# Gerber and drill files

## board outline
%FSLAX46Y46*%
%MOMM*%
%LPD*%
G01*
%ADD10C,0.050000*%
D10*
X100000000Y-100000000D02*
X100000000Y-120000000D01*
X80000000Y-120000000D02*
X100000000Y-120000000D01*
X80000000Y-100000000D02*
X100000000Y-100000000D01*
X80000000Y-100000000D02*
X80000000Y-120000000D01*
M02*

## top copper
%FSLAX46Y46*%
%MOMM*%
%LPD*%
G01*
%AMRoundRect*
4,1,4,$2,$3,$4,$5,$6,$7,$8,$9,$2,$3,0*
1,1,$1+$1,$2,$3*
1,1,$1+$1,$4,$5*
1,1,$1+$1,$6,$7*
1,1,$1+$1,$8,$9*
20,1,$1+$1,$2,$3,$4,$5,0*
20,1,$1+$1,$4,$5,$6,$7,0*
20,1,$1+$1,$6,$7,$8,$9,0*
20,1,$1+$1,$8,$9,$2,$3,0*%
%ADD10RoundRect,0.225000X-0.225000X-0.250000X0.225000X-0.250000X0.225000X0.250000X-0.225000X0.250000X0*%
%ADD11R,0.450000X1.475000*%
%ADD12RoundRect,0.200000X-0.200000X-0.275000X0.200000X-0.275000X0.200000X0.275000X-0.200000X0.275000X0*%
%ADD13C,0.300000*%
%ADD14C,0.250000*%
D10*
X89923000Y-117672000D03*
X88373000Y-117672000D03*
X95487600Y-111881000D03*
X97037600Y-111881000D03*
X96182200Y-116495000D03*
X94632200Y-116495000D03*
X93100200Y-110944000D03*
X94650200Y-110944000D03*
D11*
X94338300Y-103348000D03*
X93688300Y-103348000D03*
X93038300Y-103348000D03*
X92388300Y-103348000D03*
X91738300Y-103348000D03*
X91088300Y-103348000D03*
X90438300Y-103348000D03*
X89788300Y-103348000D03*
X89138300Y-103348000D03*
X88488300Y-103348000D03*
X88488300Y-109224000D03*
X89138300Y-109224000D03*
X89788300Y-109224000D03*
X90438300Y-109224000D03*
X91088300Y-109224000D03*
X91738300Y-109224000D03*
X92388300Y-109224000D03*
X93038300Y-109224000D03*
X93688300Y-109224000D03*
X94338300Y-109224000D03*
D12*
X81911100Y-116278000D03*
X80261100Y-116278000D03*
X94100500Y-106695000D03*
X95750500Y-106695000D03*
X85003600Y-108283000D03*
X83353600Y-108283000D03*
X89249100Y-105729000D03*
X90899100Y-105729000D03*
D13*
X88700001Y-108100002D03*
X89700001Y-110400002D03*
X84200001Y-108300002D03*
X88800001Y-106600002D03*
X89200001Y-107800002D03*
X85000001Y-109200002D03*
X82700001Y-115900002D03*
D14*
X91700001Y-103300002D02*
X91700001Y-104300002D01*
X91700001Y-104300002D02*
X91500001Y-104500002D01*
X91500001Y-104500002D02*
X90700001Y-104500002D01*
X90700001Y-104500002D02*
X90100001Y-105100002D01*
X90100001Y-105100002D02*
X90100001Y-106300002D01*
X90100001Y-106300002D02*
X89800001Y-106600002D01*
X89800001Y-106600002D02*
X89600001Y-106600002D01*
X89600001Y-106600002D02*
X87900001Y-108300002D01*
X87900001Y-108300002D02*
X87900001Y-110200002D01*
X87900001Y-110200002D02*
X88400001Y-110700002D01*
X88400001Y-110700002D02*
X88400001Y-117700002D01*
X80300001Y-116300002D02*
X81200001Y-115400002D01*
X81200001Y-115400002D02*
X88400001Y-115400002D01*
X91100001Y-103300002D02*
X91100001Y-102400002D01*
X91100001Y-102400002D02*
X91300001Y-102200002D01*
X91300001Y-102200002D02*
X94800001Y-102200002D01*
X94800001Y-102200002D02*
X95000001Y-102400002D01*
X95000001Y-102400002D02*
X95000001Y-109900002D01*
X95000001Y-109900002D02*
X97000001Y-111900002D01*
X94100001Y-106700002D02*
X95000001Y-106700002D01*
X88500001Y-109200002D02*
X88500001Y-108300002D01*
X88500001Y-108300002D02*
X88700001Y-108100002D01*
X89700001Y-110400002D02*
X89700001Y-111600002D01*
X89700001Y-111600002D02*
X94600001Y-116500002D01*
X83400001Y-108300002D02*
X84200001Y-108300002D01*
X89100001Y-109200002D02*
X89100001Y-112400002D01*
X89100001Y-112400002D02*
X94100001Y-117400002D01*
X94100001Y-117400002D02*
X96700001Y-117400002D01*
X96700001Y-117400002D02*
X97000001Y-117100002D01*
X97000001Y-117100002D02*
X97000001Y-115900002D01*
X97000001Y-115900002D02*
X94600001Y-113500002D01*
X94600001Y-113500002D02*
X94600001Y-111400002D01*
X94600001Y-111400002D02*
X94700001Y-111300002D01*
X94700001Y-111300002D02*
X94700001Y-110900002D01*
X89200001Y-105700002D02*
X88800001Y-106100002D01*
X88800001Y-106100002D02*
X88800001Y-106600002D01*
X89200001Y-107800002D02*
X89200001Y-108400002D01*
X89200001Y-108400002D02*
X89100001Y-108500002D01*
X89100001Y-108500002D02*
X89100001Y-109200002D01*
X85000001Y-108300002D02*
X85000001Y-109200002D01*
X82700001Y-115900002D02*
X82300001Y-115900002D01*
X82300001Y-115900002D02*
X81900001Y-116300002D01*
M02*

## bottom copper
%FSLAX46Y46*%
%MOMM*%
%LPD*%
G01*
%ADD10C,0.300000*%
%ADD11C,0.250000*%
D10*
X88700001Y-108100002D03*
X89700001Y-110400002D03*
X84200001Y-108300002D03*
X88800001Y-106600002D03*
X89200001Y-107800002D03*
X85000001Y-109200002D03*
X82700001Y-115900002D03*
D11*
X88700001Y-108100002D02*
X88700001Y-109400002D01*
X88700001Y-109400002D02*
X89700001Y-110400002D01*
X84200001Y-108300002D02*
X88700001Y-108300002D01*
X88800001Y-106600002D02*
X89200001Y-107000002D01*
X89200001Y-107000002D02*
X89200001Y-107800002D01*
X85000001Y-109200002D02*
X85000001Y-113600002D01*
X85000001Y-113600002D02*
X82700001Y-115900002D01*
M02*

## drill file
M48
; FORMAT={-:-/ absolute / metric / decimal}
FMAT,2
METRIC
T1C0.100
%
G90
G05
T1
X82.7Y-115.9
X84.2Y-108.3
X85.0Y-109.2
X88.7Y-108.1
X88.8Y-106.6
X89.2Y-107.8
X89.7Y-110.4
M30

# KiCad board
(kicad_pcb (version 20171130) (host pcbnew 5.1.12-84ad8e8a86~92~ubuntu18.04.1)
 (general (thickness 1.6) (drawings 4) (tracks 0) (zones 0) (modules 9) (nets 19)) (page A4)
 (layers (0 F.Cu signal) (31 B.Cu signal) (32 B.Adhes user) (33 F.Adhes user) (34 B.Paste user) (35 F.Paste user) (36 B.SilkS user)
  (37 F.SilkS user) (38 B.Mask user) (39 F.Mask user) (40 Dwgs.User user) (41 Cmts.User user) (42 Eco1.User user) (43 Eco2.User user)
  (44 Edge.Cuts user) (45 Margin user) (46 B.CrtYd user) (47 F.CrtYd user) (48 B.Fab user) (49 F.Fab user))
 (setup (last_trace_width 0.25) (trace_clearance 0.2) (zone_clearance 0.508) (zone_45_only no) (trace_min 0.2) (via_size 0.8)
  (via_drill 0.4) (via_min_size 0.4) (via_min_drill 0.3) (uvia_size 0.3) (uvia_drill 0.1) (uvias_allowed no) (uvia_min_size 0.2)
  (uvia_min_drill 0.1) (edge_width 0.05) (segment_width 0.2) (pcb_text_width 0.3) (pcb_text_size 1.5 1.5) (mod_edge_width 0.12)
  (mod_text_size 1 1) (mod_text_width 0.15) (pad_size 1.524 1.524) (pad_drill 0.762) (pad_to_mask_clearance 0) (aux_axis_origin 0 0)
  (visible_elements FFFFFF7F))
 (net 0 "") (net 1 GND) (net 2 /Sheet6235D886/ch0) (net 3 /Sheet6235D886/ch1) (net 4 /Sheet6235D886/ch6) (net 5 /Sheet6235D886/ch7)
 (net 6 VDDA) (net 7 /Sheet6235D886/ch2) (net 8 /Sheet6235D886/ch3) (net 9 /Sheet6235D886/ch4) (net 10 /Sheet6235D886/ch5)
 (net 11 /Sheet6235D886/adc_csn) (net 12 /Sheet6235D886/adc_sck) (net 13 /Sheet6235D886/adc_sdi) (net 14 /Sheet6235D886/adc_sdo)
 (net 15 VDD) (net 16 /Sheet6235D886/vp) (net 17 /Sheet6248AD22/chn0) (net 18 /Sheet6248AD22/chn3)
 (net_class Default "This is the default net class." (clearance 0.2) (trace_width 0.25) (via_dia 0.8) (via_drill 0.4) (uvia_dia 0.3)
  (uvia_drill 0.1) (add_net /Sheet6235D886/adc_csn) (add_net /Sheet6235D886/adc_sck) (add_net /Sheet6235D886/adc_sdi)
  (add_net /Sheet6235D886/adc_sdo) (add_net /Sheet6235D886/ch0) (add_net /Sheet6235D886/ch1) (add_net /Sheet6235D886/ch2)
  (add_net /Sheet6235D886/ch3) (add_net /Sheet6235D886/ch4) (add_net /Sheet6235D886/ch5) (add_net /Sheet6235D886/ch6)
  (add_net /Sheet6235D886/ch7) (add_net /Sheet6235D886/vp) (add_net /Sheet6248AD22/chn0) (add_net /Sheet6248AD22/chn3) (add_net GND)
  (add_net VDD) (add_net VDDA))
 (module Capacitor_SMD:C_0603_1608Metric (layer F.Cu) (at 89.148000 117.672000)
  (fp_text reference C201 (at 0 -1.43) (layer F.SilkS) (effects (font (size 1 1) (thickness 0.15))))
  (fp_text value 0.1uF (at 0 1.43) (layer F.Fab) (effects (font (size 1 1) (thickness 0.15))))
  (pad 2 smd roundrect (at 0.775 0) (size 0.9 0.95) (layers F.Cu F.Mask F.Paste) (roundrect_rratio 0.25) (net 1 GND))
  (pad 1 smd roundrect (at -0.775 0) (size 0.9 0.95) (layers F.Cu F.Mask F.Paste) (roundrect_rratio 0.25) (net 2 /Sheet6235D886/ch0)))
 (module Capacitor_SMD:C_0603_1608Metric (layer F.Cu) (at 96.262600 111.881000)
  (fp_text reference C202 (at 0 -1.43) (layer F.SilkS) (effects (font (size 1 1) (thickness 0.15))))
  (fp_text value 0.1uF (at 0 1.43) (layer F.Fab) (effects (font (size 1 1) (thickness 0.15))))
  (pad 1 smd roundrect (at -0.775 0) (size 0.9 0.95) (layers F.Cu F.Mask F.Paste) (roundrect_rratio 0.25) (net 1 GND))
  (pad 2 smd roundrect (at 0.775 0) (size 0.9 0.95) (layers F.Cu F.Mask F.Paste) (roundrect_rratio 0.25) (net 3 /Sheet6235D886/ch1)))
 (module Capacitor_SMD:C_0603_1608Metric (layer F.Cu) (at 95.407200 116.495000)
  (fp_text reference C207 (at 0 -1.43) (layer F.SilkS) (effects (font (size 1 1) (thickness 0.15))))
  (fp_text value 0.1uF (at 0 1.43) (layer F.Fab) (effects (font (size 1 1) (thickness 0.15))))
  (pad 2 smd roundrect (at 0.775 0) (size 0.9 0.95) (layers F.Cu F.Mask F.Paste) (roundrect_rratio 0.25) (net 1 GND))
  (pad 1 smd roundrect (at -0.775 0) (size 0.9 0.95) (layers F.Cu F.Mask F.Paste) (roundrect_rratio 0.25) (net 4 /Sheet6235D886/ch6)))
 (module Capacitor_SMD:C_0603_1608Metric (layer F.Cu) (at 93.875200 110.944000)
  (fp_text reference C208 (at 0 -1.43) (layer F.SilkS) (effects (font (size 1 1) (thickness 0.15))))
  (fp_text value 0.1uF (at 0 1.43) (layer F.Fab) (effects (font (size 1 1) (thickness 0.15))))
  (pad 1 smd roundrect (at -0.775 0) (size 0.9 0.95) (layers F.Cu F.Mask F.Paste) (roundrect_rratio 0.25) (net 1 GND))
  (pad 2 smd roundrect (at 0.775 0) (size 0.9 0.95) (layers F.Cu F.Mask F.Paste) (roundrect_rratio 0.25) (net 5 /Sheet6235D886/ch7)))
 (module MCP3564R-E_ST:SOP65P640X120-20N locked (layer F.Cu) (at 91.413300 106.286000 270.000000)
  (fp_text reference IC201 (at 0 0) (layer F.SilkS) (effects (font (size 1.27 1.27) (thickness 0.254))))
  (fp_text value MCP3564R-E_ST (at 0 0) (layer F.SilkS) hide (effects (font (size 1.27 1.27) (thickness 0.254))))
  (pad 1 smd rect (at -2.938 -2.925) (size 0.45 1.475) (layers F.Cu F.Mask F.Paste) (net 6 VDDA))
  (pad 2 smd rect (at -2.938 -2.275) (size 0.45 1.475) (layers F.Cu F.Mask F.Paste) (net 1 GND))
  (pad 3 smd rect (at -2.938 -1.625) (size 0.45 1.475) (layers F.Cu F.Mask F.Paste) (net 1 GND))
  (pad 4 smd rect (at -2.938 -0.975) (size 0.45 1.475) (layers F.Cu F.Mask F.Paste))
  (pad 5 smd rect (at -2.938 -0.325) (size 0.45 1.475) (layers F.Cu F.Mask F.Paste) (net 2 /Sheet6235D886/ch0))
  (pad 6 smd rect (at -2.938 0.325) (size 0.45 1.475) (layers F.Cu F.Mask F.Paste) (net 3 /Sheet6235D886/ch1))
  (pad 7 smd rect (at -2.938 0.975) (size 0.45 1.475) (layers F.Cu F.Mask F.Paste) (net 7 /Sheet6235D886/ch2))
  (pad 8 smd rect (at -2.938 1.625) (size 0.45 1.475) (layers F.Cu F.Mask F.Paste) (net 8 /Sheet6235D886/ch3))
  (pad 9 smd rect (at -2.938 2.275) (size 0.45 1.475) (layers F.Cu F.Mask F.Paste) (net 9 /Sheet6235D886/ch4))
  (pad 10 smd rect (at -2.938 2.925) (size 0.45 1.475) (layers F.Cu F.Mask F.Paste) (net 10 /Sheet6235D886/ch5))
  (pad 11 smd rect (at 2.938 2.925) (size 0.45 1.475) (layers F.Cu F.Mask F.Paste) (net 4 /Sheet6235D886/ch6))
  (pad 12 smd rect (at 2.938 2.275) (size 0.45 1.475) (layers F.Cu F.Mask F.Paste) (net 5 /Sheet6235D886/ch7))
  (pad 13 smd rect (at 2.938 1.625) (size 0.45 1.475) (layers F.Cu F.Mask F.Paste) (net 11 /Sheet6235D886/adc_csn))
  (pad 14 smd rect (at 2.938 0.975) (size 0.45 1.475) (layers F.Cu F.Mask F.Paste) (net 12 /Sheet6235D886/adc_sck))
  (pad 15 smd rect (at 2.938 0.325) (size 0.45 1.475) (layers F.Cu F.Mask F.Paste) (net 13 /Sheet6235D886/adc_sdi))
  (pad 16 smd rect (at 2.938 -0.325) (size 0.45 1.475) (layers F.Cu F.Mask F.Paste) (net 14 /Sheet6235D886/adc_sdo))
  (pad 17 smd rect (at 2.938 -0.975) (size 0.45 1.475) (layers F.Cu F.Mask F.Paste))
  (pad 18 smd rect (at 2.938 -1.625) (size 0.45 1.475) (layers F.Cu F.Mask F.Paste))
  (pad 19 smd rect (at 2.938 -2.275) (size 0.45 1.475) (layers F.Cu F.Mask F.Paste) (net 1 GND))
  (pad 20 smd rect (at 2.938 -2.925) (size 0.45 1.475) (layers F.Cu F.Mask F.Paste) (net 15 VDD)))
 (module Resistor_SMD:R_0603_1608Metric (layer F.Cu) (at 81.086100 116.278000)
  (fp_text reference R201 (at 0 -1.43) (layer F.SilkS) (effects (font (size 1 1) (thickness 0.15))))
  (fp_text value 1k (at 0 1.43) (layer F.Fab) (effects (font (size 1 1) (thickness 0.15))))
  (pad 2 smd roundrect (at 0.825 0) (size 0.8 0.95) (layers F.Cu F.Mask F.Paste) (roundrect_rratio 0.25) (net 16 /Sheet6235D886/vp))
  (pad 1 smd roundrect (at -0.825 0) (size 0.8 0.95) (layers F.Cu F.Mask F.Paste) (roundrect_rratio 0.25) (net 2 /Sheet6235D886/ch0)))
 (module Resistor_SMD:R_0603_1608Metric (layer F.Cu) (at 94.925500 106.695000)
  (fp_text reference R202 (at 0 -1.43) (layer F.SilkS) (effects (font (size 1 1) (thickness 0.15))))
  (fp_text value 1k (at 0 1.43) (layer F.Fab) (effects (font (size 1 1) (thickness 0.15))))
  (pad 1 smd roundrect (at -0.825 0) (size 0.8 0.95) (layers F.Cu F.Mask F.Paste) (roundrect_rratio 0.25) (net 3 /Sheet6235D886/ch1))
  (pad 2 smd roundrect (at 0.825 0) (size 0.8 0.95) (layers F.Cu F.Mask F.Paste) (roundrect_rratio 0.25) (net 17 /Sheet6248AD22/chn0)))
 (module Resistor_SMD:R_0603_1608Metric (layer F.Cu) (at 84.178600 108.283000)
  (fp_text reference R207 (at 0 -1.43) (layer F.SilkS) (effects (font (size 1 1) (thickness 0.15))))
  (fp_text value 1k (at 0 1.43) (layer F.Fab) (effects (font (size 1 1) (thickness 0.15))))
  (pad 2 smd roundrect (at 0.825 0) (size 0.8 0.95) (layers F.Cu F.Mask F.Paste) (roundrect_rratio 0.25) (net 16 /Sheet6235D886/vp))
  (pad 1 smd roundrect (at -0.825 0) (size 0.8 0.95) (layers F.Cu F.Mask F.Paste) (roundrect_rratio 0.25) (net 4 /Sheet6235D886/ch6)))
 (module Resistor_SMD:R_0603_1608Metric (layer F.Cu) (at 90.074100 105.729000)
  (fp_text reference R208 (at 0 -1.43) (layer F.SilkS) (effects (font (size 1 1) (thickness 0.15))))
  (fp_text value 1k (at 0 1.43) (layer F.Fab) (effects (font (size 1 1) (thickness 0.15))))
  (pad 1 smd roundrect (at -0.825 0) (size 0.8 0.95) (layers F.Cu F.Mask F.Paste) (roundrect_rratio 0.25) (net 5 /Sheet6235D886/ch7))
  (pad 2 smd roundrect (at 0.825 0) (size 0.8 0.95) (layers F.Cu F.Mask F.Paste) (roundrect_rratio 0.25) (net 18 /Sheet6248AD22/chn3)))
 (gr_line (start 100 100) (end 100 120) (layer Edge.Cuts) (width 0.05))
 (gr_line (start 80 120) (end 100 120) (layer Edge.Cuts) (width 0.05))
 (gr_line (start 80 100) (end 100 100) (layer Edge.Cuts) (width 0.05))
 (gr_line (start 80 100) (end 80 120) (layer Edge.Cuts) (width 0.05))
 (segment (start 91.700001 103.300002) (end 91.700001 104.300002) (width 0.250000) (layer F.Cu) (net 2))
 (segment (start 91.700001 104.300002) (end 91.500001 104.500002) (width 0.250000) (layer F.Cu) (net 2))
 (segment (start 91.500001 104.500002) (end 90.700001 104.500002) (width 0.250000) (layer F.Cu) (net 2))
 (segment (start 90.700001 104.500002) (end 90.100001 105.100002) (width 0.250000) (layer F.Cu) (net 2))
 (segment (start 90.100001 105.100002) (end 90.100001 106.300002) (width 0.250000) (layer F.Cu) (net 2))
 (segment (start 90.100001 106.300002) (end 89.800001 106.600002) (width 0.250000) (layer F.Cu) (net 2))
 (segment (start 89.800001 106.600002) (end 89.600001 106.600002) (width 0.250000) (layer F.Cu) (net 2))
 (segment (start 89.600001 106.600002) (end 87.900001 108.300002) (width 0.250000) (layer F.Cu) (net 2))
 (segment (start 87.900001 108.300002) (end 87.900001 110.200002) (width 0.250000) (layer F.Cu) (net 2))
 (segment (start 87.900001 110.200002) (end 88.400001 110.700002) (width 0.250000) (layer F.Cu) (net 2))
 (segment (start 88.400001 110.700002) (end 88.400001 117.700002) (width 0.250000) (layer F.Cu) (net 2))
 (segment (start 80.300001 116.300002) (end 81.200001 115.400002) (width 0.250000) (layer F.Cu) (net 2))
 (segment (start 81.200001 115.400002) (end 88.400001 115.400002) (width 0.250000) (layer F.Cu) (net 2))
 (segment (start 91.100001 103.300002) (end 91.100001 102.400002) (width 0.250000) (layer F.Cu) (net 3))
 (segment (start 91.100001 102.400002) (end 91.300001 102.200002) (width 0.250000) (layer F.Cu) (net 3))
 (segment (start 91.300001 102.200002) (end 94.800001 102.200002) (width 0.250000) (layer F.Cu) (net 3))
 (segment (start 94.800001 102.200002) (end 95.000001 102.400002) (width 0.250000) (layer F.Cu) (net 3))
 (segment (start 95.000001 102.400002) (end 95.000001 109.900002) (width 0.250000) (layer F.Cu) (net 3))
 (segment (start 95.000001 109.900002) (end 97.000001 111.900002) (width 0.250000) (layer F.Cu) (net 3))
 (segment (start 94.100001 106.700002) (end 95.000001 106.700002) (width 0.250000) (layer F.Cu) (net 3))
 (segment (start 88.500001 109.200002) (end 88.500001 108.300002) (width 0.250000) (layer F.Cu) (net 4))
 (segment (start 88.500001 108.300002) (end 88.700001 108.100002) (width 0.250000) (layer F.Cu) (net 4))
 (segment (start 88.700001 108.100002) (end 88.700001 109.400002) (width 0.250000) (layer B.Cu) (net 4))
 (segment (start 88.700001 109.400002) (end 89.700001 110.400002) (width 0.250000) (layer B.Cu) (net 4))
 (segment (start 89.700001 110.400002) (end 89.700001 111.600002) (width 0.250000) (layer F.Cu) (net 4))
 (segment (start 89.700001 111.600002) (end 94.600001 116.500002) (width 0.250000) (layer F.Cu) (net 4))
 (segment (start 83.400001 108.300002) (end 84.200001 108.300002) (width 0.250000) (layer F.Cu) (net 4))
 (segment (start 84.200001 108.300002) (end 88.700001 108.300002) (width 0.250000) (layer B.Cu) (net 4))
 (via micro (at 88.700001 108.100002) (size 0.300000) (drill 0.100000) (layers F.Cu B.Cu) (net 4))
 (via micro (at 89.700001 110.400002) (size 0.300000) (drill 0.100000) (layers F.Cu B.Cu) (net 4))
 (via micro (at 84.200001 108.300002) (size 0.300000) (drill 0.100000) (layers F.Cu B.Cu) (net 4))
 (segment (start 89.100001 109.200002) (end 89.100001 112.400002) (width 0.250000) (layer F.Cu) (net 5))
 (segment (start 89.100001 112.400002) (end 94.100001 117.400002) (width 0.250000) (layer F.Cu) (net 5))
 (segment (start 94.100001 117.400002) (end 96.700001 117.400002) (width 0.250000) (layer F.Cu) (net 5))
 (segment (start 96.700001 117.400002) (end 97.000001 117.100002) (width 0.250000) (layer F.Cu) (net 5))
 (segment (start 97.000001 117.100002) (end 97.000001 115.900002) (width 0.250000) (layer F.Cu) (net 5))
 (segment (start 97.000001 115.900002) (end 94.600001 113.500002) (width 0.250000) (layer F.Cu) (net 5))
 (segment (start 94.600001 113.500002) (end 94.600001 111.400002) (width 0.250000) (layer F.Cu) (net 5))
 (segment (start 94.600001 111.400002) (end 94.700001 111.300002) (width 0.250000) (layer F.Cu) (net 5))
 (segment (start 94.700001 111.300002) (end 94.700001 110.900002) (width 0.250000) (layer F.Cu) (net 5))
 (segment (start 89.200001 105.700002) (end 88.800001 106.100002) (width 0.250000) (layer F.Cu) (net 5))
 (segment (start 88.800001 106.100002) (end 88.800001 106.600002) (width 0.250000) (layer F.Cu) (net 5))
 (segment (start 88.800001 106.600002) (end 89.200001 107.000002) (width 0.250000) (layer B.Cu) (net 5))
 (segment (start 89.200001 107.000002) (end 89.200001 107.800002) (width 0.250000) (layer B.Cu) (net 5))
 (segment (start 89.200001 107.800002) (end 89.200001 108.400002) (width 0.250000) (layer F.Cu) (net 5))
 (segment (start 89.200001 108.400002) (end 89.100001 108.500002) (width 0.250000) (layer F.Cu) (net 5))
 (segment (start 89.100001 108.500002) (end 89.100001 109.200002) (width 0.250000) (layer F.Cu) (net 5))
 (via micro (at 88.800001 106.600002) (size 0.300000) (drill 0.100000) (layers F.Cu B.Cu) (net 5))
 (via micro (at 89.200001 107.800002) (size 0.300000) (drill 0.100000) (layers F.Cu B.Cu) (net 5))
 (segment (start 85.000001 108.300002) (end 85.000001 109.200002) (width 0.250000) (layer F.Cu) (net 16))
 (segment (start 85.000001 109.200002) (end 85.000001 113.600002) (width 0.250000) (layer B.Cu) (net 16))
 (segment (start 85.000001 113.600002) (end 82.700001 115.900002) (width 0.250000) (layer B.Cu) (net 16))
 (segment (start 82.700001 115.900002) (end 82.300001 115.900002) (width 0.250000) (layer F.Cu) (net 16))
 (segment (start 82.300001 115.900002) (end 81.900001 116.300002) (width 0.250000) (layer F.Cu) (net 16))
 (via micro (at 85.000001 109.200002) (size 0.300000) (drill 0.100000) (layers F.Cu B.Cu) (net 16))
 (via micro (at 82.700001 115.900002) (size 0.300000) (drill 0.100000) (layers F.Cu B.Cu) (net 16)))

